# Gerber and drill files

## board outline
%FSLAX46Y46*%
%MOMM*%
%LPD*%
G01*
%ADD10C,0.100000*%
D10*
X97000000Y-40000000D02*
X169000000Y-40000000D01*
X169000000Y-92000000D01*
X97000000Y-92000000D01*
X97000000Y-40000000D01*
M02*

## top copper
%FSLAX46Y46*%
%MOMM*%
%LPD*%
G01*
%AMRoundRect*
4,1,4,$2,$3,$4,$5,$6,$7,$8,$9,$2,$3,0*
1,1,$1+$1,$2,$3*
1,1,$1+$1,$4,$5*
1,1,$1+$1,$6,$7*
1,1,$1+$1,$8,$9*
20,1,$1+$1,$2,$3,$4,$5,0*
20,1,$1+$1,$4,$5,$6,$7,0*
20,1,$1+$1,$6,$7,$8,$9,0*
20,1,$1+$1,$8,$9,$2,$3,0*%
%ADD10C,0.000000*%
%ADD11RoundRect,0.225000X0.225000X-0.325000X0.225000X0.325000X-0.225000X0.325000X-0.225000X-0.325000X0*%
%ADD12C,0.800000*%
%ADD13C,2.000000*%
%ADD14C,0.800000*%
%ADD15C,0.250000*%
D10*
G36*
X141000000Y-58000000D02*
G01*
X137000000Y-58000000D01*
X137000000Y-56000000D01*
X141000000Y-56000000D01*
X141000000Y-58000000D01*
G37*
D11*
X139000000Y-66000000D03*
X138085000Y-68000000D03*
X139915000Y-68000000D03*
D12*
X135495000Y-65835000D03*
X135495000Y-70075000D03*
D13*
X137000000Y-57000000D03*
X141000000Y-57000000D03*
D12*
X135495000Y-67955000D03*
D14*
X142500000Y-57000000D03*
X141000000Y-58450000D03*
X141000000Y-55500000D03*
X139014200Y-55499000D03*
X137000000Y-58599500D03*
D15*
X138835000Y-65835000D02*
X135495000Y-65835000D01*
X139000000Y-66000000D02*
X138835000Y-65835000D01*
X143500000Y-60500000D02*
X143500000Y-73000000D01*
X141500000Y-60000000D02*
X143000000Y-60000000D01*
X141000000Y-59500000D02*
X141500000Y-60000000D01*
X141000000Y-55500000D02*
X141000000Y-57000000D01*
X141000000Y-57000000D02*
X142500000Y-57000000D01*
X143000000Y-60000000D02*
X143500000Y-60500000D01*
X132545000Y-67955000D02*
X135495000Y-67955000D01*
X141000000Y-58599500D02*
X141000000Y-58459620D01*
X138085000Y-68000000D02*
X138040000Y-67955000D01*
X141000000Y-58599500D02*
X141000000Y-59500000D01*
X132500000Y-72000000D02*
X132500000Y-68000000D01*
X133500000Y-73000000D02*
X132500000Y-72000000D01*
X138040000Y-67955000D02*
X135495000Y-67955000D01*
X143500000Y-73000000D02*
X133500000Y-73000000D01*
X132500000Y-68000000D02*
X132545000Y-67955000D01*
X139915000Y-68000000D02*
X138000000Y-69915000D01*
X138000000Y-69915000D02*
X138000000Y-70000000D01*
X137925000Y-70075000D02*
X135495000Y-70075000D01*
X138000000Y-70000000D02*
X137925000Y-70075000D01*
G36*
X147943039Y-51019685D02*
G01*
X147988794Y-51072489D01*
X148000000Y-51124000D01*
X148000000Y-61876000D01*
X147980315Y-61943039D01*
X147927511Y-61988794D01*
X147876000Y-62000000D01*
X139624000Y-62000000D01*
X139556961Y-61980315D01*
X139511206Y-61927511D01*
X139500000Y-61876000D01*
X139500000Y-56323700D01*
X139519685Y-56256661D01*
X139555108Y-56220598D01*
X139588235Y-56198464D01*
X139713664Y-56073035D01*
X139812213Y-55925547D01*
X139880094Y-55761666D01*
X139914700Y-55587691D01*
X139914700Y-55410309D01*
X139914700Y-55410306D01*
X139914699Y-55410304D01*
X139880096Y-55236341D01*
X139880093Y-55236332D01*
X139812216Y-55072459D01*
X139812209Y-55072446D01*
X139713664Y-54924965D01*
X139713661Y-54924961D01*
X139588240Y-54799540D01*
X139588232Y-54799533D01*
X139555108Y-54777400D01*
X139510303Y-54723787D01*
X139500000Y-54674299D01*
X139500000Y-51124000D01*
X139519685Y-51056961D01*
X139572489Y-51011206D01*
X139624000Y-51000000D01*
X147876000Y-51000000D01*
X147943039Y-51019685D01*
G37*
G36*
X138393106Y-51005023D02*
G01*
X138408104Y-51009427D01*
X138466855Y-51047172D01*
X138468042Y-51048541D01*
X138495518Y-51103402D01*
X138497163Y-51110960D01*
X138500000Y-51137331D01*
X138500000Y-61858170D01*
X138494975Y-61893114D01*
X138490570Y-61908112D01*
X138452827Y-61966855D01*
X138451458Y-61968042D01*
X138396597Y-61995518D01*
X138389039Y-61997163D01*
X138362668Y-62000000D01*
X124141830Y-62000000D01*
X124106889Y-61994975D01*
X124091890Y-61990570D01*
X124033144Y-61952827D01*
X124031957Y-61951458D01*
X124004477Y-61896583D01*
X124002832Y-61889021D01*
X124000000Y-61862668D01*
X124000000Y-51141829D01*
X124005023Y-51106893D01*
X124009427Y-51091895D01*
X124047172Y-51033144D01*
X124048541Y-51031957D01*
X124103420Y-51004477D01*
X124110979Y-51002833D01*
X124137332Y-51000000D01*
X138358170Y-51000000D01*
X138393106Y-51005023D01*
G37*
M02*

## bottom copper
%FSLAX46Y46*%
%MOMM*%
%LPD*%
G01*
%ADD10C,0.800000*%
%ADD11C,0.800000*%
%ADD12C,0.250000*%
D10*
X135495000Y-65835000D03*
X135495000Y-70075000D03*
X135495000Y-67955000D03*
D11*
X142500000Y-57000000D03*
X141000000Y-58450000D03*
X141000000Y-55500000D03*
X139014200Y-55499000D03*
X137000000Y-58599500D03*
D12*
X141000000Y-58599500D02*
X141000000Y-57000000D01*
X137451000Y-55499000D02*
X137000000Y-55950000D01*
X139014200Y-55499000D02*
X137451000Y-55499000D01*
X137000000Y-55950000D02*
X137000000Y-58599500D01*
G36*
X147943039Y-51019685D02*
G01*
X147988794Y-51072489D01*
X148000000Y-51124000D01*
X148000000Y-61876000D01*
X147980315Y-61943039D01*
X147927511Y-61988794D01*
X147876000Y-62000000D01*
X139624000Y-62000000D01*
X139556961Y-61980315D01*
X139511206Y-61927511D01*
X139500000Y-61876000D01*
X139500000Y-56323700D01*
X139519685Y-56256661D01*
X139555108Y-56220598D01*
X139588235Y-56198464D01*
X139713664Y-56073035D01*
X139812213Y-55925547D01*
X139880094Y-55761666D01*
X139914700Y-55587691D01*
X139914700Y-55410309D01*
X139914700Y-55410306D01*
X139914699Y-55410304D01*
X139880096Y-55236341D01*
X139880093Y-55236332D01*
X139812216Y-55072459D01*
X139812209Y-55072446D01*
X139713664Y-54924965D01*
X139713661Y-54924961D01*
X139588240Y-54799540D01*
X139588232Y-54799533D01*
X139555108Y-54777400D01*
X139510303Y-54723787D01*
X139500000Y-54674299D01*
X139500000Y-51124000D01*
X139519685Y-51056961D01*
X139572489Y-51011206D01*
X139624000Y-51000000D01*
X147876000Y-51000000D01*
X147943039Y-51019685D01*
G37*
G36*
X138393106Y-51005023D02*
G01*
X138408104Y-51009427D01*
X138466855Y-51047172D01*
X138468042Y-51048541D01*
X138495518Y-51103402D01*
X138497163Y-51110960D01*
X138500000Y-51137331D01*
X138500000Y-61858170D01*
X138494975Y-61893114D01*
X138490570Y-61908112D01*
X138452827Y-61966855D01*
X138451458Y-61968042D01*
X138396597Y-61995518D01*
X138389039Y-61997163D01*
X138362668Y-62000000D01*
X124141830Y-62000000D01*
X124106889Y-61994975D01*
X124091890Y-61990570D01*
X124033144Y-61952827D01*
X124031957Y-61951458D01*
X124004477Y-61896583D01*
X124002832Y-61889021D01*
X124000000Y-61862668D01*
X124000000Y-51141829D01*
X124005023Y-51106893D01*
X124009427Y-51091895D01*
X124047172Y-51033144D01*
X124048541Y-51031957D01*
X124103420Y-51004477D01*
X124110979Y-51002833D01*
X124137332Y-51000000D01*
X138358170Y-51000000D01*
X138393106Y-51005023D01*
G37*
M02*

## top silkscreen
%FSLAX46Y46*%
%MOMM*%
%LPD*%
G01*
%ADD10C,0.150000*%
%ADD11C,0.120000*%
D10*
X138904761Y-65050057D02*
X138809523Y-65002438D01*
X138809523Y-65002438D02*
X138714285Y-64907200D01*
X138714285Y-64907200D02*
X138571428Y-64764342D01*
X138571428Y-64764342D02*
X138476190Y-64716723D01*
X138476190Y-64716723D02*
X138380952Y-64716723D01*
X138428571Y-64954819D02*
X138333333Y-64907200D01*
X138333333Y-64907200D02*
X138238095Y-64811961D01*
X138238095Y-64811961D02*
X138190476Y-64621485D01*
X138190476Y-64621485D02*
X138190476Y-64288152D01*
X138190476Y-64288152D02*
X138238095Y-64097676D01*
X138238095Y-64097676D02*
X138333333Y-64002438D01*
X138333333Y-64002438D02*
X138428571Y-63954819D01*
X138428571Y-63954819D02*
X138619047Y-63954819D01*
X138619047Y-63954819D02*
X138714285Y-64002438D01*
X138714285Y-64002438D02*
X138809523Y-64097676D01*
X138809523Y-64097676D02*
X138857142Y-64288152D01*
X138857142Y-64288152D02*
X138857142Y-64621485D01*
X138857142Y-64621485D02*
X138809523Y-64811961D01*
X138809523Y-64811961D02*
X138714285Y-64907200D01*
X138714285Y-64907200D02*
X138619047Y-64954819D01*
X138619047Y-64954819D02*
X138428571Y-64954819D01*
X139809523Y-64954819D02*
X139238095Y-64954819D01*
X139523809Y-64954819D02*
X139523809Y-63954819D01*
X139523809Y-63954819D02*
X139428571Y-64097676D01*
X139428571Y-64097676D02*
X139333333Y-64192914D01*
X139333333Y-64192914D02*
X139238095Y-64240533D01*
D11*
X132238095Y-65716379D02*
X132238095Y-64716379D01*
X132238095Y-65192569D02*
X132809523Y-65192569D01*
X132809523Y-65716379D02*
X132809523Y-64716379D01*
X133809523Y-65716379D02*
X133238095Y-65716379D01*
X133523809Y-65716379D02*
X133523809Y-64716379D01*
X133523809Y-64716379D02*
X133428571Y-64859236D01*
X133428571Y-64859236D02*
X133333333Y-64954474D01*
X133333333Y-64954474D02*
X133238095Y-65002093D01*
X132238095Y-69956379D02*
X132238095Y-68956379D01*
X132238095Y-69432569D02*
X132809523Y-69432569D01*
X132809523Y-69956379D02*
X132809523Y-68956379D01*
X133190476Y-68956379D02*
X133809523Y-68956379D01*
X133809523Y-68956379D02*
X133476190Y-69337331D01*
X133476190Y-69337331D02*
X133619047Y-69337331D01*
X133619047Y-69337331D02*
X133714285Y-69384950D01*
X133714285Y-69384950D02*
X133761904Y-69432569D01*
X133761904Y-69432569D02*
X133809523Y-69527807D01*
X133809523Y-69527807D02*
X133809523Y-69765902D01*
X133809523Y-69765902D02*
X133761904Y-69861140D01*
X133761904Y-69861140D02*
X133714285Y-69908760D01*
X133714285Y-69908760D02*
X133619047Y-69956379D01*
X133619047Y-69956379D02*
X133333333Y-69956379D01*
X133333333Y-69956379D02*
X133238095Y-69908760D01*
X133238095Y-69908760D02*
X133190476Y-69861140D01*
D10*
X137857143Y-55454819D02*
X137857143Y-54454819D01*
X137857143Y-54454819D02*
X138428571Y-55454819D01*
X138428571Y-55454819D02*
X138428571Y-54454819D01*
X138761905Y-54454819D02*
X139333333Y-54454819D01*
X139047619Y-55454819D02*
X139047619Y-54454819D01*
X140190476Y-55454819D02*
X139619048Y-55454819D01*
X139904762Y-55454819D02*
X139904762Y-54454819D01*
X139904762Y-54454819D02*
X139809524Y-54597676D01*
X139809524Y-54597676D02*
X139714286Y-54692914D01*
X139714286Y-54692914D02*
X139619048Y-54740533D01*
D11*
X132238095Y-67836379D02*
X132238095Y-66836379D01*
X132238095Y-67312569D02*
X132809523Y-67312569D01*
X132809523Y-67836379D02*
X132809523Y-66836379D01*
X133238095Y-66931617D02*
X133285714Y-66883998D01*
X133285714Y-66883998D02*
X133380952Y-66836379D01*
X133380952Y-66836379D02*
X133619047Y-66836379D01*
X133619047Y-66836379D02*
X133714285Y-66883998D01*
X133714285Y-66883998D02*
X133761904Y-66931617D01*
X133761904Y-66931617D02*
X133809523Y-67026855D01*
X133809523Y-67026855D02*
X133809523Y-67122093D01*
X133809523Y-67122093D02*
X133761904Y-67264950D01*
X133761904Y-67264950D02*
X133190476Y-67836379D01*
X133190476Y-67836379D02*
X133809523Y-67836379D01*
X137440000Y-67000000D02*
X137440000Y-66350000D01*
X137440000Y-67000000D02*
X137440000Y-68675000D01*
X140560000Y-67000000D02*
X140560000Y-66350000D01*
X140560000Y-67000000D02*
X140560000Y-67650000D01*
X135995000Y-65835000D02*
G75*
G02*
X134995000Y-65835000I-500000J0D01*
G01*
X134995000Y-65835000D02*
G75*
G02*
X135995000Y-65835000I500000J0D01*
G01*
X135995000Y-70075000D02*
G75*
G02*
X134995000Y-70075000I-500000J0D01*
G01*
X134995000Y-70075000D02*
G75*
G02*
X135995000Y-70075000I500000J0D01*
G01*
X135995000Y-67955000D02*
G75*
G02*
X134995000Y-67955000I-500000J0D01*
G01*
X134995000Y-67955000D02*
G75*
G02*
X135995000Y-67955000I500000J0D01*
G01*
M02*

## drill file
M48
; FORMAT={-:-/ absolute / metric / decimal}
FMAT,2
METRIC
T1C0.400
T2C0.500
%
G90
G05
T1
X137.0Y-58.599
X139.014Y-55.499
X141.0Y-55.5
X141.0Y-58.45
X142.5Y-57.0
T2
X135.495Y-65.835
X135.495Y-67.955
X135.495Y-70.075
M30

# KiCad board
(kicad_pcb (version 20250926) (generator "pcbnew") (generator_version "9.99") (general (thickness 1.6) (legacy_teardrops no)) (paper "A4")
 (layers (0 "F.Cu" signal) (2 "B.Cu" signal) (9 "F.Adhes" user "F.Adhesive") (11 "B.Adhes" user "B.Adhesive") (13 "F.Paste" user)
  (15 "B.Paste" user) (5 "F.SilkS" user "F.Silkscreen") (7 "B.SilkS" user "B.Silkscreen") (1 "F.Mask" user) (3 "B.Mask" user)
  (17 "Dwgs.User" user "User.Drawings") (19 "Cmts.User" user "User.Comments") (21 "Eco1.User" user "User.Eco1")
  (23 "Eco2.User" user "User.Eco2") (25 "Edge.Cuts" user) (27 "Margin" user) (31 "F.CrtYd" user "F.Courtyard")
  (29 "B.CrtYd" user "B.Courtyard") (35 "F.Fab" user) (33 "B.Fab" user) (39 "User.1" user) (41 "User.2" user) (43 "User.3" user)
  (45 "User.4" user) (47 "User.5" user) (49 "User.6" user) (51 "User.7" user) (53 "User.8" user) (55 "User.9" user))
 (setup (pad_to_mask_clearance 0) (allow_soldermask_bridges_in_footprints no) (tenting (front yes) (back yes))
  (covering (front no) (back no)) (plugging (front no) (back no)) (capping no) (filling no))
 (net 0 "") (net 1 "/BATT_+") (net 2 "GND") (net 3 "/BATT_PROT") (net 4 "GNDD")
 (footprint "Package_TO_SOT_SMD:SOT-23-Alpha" (layer "F.Cu") (at 139 67 90)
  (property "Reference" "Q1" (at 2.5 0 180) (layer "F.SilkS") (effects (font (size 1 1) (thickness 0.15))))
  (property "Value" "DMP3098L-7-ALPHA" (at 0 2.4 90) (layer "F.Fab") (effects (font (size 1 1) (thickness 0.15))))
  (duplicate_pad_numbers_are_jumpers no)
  (fp_line (start 0 -1.56) (end 0.65 -1.56) (stroke (width 0.12) (type solid)) (layer "F.SilkS"))
  (fp_line (start 0 -1.56) (end -1.675 -1.56) (stroke (width 0.12) (type solid)) (layer "F.SilkS"))
  (fp_line (start 0 1.56) (end 0.65 1.56) (stroke (width 0.12) (type solid)) (layer "F.SilkS"))
  (fp_line (start 0 1.56) (end -0.65 1.56) (stroke (width 0.12) (type solid)) (layer "F.SilkS"))
  (pad "D" smd roundrect (at 1 0 90) (size 1.1 0.9) (layers "F.Cu" "F.Mask" "F.Paste") (roundrect_rratio 0.25) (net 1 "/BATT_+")
   (tenting (front none) (back none)))
  (pad "G" smd roundrect (at -1 -0.915 90) (size 1.1 0.9) (layers "F.Cu" "F.Mask" "F.Paste") (roundrect_rratio 0.25) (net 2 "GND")
   (tenting (front none) (back none)))
  (pad "S" smd roundrect (at -1 0.915 90) (size 1.1 0.9) (layers "F.Cu" "F.Mask" "F.Paste") (roundrect_rratio 0.25) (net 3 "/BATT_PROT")
   (tenting (front none) (back none))))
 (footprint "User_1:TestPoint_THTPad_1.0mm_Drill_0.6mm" (layer "F.Cu") (at 135.495 65.835)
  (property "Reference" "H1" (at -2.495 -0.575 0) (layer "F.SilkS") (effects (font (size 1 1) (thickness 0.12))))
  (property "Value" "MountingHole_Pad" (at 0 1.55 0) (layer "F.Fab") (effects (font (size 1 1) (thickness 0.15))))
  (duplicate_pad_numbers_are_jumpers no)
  (fp_circle (center 0 0) (end 0.5 0) (stroke (width 0.12) (type solid)) (fill no) (layer "F.SilkS"))
  (pad "1" thru_hole circle (at 0 0) (size 0.8 0.8) (drill 0.5) (layers "*.Cu" "*.Mask") (remove_unused_layers no) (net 1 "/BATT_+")
   (tenting (front none) (back none))))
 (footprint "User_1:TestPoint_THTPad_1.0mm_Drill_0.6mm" (layer "F.Cu") (at 135.495 70.075)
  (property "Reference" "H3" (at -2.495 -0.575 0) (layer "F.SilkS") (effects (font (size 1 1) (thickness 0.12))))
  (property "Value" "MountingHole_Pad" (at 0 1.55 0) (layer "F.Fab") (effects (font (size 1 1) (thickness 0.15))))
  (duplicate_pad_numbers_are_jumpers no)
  (fp_circle (center 0 0) (end 0.5 0) (stroke (width 0.12) (type solid)) (fill no) (layer "F.SilkS"))
  (pad "1" thru_hole circle (at 0 0) (size 0.8 0.8) (drill 0.5) (layers "*.Cu" "*.Mask") (remove_unused_layers no) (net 3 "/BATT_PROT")
   (tenting (front none) (back none))))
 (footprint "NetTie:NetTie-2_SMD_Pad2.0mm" (layer "F.Cu") (at 139 57)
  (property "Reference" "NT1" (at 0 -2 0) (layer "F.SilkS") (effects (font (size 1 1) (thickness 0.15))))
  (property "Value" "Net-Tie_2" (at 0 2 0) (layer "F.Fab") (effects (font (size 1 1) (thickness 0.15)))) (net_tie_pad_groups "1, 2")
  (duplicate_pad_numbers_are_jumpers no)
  (fp_poly (pts (xy -2 -1) (xy 2 -1) (xy 2 1) (xy -2 1)) (stroke (width 0) (type solid)) (fill yes) (layer "F.Cu"))
  (pad "1" smd circle (at -2 0) (size 2 2) (layers "F.Cu") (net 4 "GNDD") (tenting (front none) (back none)))
  (pad "2" smd circle (at 2 0) (size 2 2) (layers "F.Cu") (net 2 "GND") (tenting (front none) (back none))))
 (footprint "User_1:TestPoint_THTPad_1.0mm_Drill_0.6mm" (layer "F.Cu") (at 135.495 67.955)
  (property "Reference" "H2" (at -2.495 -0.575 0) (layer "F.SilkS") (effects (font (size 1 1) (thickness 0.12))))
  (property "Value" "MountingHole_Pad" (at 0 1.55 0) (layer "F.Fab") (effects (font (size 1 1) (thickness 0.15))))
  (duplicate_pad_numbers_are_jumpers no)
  (fp_circle (center 0 0) (end 0.5 0) (stroke (width 0.12) (type solid)) (fill no) (layer "F.SilkS"))
  (pad "1" thru_hole circle (at 0 0) (size 0.8 0.8) (drill 0.5) (layers "*.Cu" "*.Mask") (remove_unused_layers no) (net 2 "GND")
   (tenting (front none) (back none))))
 (gr_rect (start 97 40) (end 169 92) (stroke (width 0.1) (type default)) (fill no) (layer "Edge.Cuts"))
 (segment (start 138.835 65.835) (end 135.495 65.835) (width 0.25) (layer "F.Cu") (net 1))
 (segment (start 139 66) (end 138.835 65.835) (width 0.25) (layer "F.Cu") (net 1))
 (segment (start 143.5 60.5) (end 143.5 73) (width 0.25) (layer "F.Cu") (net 2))
 (segment (start 141.5 60) (end 143 60) (width 0.25) (layer "F.Cu") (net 2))
 (segment (start 141 59.5) (end 141.5 60) (width 0.25) (layer "F.Cu") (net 2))
 (segment (start 141 55.5) (end 141 57) (width 0.25) (layer "F.Cu") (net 2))
 (segment (start 141 57) (end 142.5 57) (width 0.25) (layer "F.Cu") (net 2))
 (segment (start 143 60) (end 143.5 60.5) (width 0.25) (layer "F.Cu") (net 2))
 (segment (start 132.545 67.955) (end 135.495 67.955) (width 0.25) (layer "F.Cu") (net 2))
 (segment (start 141 58.5995) (end 141 58.45962) (width 0.25) (layer "F.Cu") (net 2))
 (segment (start 138.085 68) (end 138.04 67.955) (width 0.25) (layer "F.Cu") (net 2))
 (segment (start 141 58.5995) (end 141 59.5) (width 0.25) (layer "F.Cu") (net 2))
 (segment (start 132.5 72) (end 132.5 68) (width 0.25) (layer "F.Cu") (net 2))
 (segment (start 133.5 73) (end 132.5 72) (width 0.25) (layer "F.Cu") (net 2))
 (segment (start 138.04 67.955) (end 135.495 67.955) (width 0.25) (layer "F.Cu") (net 2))
 (segment (start 143.5 73) (end 133.5 73) (width 0.25) (layer "F.Cu") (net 2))
 (segment (start 132.5 68) (end 132.545 67.955) (width 0.25) (layer "F.Cu") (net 2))
 (via (at 142.5 57) (size 0.8) (drill 0.4) (layers "F.Cu" "B.Cu") (tenting (front none) (back none)) (capping none)
  (covering (front none) (back none)) (plugging (front none) (back none)) (filling none) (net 2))
 (via (at 141 58.45) (size 0.8) (drill 0.4) (layers "F.Cu" "B.Cu") (tenting (front none) (back none)) (capping none)
  (covering (front none) (back none)) (plugging (front none) (back none)) (filling none) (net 2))
 (via (at 141 55.5) (size 0.8) (drill 0.4) (layers "F.Cu" "B.Cu") (tenting (front none) (back none)) (capping none)
  (covering (front none) (back none)) (plugging (front none) (back none)) (filling none) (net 2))
 (segment (start 141 58.5995) (end 141 57) (width 0.25) (layer "B.Cu") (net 2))
 (segment (start 139.915 68) (end 138 69.915) (width 0.25) (layer "F.Cu") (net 3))
 (segment (start 138 69.915) (end 138 70) (width 0.25) (layer "F.Cu") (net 3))
 (segment (start 137.925 70.075) (end 135.495 70.075) (width 0.25) (layer "F.Cu") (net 3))
 (segment (start 138 70) (end 137.925 70.075) (width 0.25) (layer "F.Cu") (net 3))
 (via (at 139.0142 55.499) (size 0.8) (drill 0.4) (layers "F.Cu" "B.Cu") (tenting (front none) (back none)) (capping none)
  (covering (front none) (back none)) (plugging (front none) (back none)) (filling none) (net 4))
 (via (at 137 58.5995) (size 0.8) (drill 0.4) (layers "F.Cu" "B.Cu") (tenting (front none) (back none)) (capping none)
  (covering (front none) (back none)) (plugging (front none) (back none)) (filling none) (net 4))
 (segment (start 137.451 55.499) (end 137 55.95) (width 0.25) (layer "B.Cu") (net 4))
 (segment (start 139.0142 55.499) (end 137.451 55.499) (width 0.25) (layer "B.Cu") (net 4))
 (segment (start 137 55.95) (end 137 58.5995) (width 0.25) (layer "B.Cu") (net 4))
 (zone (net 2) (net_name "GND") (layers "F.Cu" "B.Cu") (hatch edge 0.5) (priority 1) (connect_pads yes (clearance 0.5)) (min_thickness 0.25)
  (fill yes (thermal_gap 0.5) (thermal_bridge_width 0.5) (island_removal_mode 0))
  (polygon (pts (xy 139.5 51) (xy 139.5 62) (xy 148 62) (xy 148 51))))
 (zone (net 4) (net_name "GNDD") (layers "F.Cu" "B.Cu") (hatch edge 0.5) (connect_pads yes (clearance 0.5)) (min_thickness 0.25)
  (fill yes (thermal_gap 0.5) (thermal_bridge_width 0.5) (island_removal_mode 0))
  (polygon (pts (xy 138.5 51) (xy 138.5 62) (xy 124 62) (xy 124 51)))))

